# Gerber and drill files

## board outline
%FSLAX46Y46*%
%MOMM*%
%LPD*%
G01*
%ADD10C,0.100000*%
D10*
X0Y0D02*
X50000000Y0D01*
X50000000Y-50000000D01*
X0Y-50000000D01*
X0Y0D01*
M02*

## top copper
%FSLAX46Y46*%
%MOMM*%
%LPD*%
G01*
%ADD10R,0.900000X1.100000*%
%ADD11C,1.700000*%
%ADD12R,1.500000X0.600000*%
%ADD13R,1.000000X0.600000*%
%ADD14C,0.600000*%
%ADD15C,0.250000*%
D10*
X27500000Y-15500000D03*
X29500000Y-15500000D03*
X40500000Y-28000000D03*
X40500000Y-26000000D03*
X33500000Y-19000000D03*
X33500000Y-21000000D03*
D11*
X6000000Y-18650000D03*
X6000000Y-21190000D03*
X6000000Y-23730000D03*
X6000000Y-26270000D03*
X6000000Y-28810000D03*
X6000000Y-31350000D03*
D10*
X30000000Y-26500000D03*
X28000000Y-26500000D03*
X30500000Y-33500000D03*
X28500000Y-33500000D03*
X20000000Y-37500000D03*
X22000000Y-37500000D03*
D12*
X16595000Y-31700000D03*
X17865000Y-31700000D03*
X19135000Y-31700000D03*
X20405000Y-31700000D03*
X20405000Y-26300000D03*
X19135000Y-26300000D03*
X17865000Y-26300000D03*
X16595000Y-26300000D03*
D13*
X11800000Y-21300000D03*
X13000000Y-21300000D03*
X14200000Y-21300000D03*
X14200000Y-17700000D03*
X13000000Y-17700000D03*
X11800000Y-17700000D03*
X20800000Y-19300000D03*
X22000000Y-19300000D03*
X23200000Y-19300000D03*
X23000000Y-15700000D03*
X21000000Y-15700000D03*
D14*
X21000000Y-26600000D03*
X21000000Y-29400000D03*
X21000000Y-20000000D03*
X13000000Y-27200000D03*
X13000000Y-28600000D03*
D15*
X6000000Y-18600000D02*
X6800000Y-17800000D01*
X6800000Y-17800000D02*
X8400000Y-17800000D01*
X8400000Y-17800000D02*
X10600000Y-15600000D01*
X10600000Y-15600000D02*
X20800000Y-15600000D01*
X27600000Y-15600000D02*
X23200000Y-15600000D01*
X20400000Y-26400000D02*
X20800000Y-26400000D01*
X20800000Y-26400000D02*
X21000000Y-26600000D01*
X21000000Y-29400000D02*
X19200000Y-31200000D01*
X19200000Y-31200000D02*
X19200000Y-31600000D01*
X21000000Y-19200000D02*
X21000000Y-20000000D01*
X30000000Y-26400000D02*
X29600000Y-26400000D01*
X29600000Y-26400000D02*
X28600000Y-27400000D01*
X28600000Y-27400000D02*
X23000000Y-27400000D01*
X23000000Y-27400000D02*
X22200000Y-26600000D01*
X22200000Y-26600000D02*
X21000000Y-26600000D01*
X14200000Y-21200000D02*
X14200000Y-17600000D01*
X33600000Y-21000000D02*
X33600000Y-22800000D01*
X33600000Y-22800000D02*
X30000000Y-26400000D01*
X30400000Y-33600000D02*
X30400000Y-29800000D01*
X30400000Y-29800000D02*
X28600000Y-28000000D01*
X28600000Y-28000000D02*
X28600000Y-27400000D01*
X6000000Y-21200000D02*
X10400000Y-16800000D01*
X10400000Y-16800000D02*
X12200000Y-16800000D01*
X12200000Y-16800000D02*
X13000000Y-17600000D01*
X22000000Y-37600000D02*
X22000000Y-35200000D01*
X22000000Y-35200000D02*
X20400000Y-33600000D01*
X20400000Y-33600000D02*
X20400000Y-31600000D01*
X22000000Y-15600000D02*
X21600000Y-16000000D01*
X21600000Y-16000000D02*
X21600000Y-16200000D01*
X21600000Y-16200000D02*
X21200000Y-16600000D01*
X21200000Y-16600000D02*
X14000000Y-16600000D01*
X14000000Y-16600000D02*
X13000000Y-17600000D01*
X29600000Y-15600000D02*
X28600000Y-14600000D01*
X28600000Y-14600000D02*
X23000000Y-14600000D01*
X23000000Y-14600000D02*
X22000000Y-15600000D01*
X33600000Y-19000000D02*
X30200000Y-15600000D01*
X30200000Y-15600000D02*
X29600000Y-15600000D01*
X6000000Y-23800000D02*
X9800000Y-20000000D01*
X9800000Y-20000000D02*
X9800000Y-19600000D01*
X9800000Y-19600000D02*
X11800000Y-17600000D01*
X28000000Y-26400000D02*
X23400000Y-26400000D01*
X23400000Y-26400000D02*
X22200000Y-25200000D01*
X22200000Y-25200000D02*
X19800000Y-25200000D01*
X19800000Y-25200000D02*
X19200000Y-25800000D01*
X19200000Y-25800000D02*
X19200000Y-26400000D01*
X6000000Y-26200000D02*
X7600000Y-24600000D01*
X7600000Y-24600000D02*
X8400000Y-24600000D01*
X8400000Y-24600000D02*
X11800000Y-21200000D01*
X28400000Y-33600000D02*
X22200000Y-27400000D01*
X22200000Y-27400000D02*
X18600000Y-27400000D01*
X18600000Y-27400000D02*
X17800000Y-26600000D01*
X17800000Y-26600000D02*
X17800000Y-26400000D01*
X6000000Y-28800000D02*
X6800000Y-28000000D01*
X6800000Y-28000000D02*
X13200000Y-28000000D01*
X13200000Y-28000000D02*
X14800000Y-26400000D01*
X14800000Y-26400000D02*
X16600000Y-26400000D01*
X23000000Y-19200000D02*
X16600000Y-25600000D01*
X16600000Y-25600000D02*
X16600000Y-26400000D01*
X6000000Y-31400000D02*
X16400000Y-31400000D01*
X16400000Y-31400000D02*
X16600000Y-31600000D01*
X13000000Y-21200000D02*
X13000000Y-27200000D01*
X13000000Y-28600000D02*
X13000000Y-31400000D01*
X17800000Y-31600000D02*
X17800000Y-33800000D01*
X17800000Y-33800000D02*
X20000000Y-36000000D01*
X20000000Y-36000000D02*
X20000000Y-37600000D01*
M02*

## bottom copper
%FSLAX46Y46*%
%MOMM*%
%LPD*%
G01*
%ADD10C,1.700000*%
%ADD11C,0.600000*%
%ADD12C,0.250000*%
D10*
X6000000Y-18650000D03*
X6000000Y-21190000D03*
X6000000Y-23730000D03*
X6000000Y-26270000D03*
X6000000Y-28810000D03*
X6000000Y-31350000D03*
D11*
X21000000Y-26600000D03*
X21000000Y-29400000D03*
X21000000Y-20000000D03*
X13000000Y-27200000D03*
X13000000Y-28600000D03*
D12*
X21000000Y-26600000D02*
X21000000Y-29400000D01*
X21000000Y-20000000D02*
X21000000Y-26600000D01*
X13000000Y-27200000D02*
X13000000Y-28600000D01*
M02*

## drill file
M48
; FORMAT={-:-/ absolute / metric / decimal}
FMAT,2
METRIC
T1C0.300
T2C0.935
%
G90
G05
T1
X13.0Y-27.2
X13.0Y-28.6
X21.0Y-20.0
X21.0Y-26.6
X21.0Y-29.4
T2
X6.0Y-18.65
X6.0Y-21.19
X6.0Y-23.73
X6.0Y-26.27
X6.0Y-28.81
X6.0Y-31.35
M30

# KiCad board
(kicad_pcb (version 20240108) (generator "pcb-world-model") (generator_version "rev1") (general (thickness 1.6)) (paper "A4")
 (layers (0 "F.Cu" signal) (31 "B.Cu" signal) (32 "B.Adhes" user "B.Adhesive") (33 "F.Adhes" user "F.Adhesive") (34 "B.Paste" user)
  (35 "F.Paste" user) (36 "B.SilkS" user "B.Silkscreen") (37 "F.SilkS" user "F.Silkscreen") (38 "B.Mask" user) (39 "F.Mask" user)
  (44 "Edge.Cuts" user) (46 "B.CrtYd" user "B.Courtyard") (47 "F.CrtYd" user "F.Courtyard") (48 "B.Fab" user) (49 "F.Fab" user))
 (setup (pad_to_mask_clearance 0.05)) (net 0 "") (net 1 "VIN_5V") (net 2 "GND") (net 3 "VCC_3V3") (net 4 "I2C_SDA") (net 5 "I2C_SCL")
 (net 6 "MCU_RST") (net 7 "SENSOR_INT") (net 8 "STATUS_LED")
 (gr_rect (start 0.0 0.0) (end 50.0000 50.0000) (stroke (width 0.1) (type default)) (fill none) (layer "Edge.Cuts"))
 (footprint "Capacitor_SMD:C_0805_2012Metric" (layer "F.Cu") (at 28.5000 15.5000 0)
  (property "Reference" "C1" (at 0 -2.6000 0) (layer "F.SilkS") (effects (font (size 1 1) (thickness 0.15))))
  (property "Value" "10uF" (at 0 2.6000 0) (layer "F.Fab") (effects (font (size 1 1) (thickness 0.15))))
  (pad "1" smd rect (at -1.0000 0.0000) (size 0.9000 1.1000) (layers "F.Cu" "F.Paste" "F.Mask") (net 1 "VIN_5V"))
  (pad "2" smd rect (at 1.0000 0.0000) (size 0.9000 1.1000) (layers "F.Cu" "F.Paste" "F.Mask") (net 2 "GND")))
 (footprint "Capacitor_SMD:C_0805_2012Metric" (layer "F.Cu") (at 40.5000 27.0000 90)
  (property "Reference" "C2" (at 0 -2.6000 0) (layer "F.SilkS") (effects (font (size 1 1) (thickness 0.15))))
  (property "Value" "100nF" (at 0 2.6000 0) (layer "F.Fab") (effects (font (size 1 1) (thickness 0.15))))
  (pad "1" smd rect (at -1.0000 0.0000) (size 0.9000 1.1000) (layers "F.Cu" "F.Paste" "F.Mask") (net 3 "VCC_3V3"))
  (pad "2" smd rect (at 1.0000 0.0000) (size 0.9000 1.1000) (layers "F.Cu" "F.Paste" "F.Mask") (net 2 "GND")))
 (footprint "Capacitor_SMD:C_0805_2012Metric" (layer "F.Cu") (at 33.5000 20.0000 270)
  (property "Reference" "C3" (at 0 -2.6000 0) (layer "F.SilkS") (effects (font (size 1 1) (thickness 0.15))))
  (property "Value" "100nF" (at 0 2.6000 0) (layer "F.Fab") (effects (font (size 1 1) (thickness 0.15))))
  (pad "1" smd rect (at -1.0000 0.0000) (size 0.9000 1.1000) (layers "F.Cu" "F.Paste" "F.Mask") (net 3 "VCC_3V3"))
  (pad "2" smd rect (at 1.0000 0.0000) (size 0.9000 1.1000) (layers "F.Cu" "F.Paste" "F.Mask") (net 2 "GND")))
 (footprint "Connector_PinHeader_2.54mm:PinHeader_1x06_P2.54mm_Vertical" (layer "F.Cu") (at 6.0000 25.0000 0) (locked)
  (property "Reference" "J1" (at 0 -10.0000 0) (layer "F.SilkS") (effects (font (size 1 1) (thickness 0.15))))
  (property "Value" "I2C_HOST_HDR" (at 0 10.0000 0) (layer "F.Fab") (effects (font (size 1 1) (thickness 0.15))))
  (pad "1" thru_hole circle (at 0.0000 -6.3500) (size 1.7000 1.7000) (drill 0.9350) (layers "*.Cu" "*.Mask") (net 1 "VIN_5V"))
  (pad "2" thru_hole circle (at 0.0000 -3.8100) (size 1.7000 1.7000) (drill 0.9350) (layers "*.Cu" "*.Mask") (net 2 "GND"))
  (pad "3" thru_hole circle (at 0.0000 -1.2700) (size 1.7000 1.7000) (drill 0.9350) (layers "*.Cu" "*.Mask") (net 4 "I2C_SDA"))
  (pad "4" thru_hole circle (at 0.0000 1.2700) (size 1.7000 1.7000) (drill 0.9350) (layers "*.Cu" "*.Mask") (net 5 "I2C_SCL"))
  (pad "5" thru_hole circle (at 0.0000 3.8100) (size 1.7000 1.7000) (drill 0.9350) (layers "*.Cu" "*.Mask") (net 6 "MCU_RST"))
  (pad "6" thru_hole circle (at 0.0000 6.3500) (size 1.7000 1.7000) (drill 0.9350) (layers "*.Cu" "*.Mask") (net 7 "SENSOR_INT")))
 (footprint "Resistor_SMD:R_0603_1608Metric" (layer "F.Cu") (at 29.0000 26.5000 180)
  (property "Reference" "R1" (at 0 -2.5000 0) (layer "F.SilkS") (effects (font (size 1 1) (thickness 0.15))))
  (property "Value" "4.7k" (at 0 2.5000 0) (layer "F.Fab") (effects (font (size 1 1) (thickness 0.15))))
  (pad "1" smd rect (at -1.0000 0.0000) (size 0.9000 1.1000) (layers "F.Cu" "F.Paste" "F.Mask") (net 3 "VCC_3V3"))
  (pad "2" smd rect (at 1.0000 0.0000) (size 0.9000 1.1000) (layers "F.Cu" "F.Paste" "F.Mask") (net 4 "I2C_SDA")))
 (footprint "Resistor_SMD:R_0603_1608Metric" (layer "F.Cu") (at 29.5000 33.5000 180)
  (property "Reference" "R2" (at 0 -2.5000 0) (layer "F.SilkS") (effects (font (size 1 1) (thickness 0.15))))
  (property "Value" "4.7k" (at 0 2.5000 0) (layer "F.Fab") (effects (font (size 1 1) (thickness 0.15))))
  (pad "1" smd rect (at -1.0000 0.0000) (size 0.9000 1.1000) (layers "F.Cu" "F.Paste" "F.Mask") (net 3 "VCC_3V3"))
  (pad "2" smd rect (at 1.0000 0.0000) (size 0.9000 1.1000) (layers "F.Cu" "F.Paste" "F.Mask") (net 5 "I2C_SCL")))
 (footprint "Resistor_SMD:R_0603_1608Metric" (layer "F.Cu") (at 21.0000 37.5000 0)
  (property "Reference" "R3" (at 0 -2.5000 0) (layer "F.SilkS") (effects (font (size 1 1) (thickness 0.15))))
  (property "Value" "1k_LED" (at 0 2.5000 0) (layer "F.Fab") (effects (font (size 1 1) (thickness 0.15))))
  (pad "1" smd rect (at -1.0000 0.0000) (size 0.9000 1.1000) (layers "F.Cu" "F.Paste" "F.Mask") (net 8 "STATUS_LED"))
  (pad "2" smd rect (at 1.0000 0.0000) (size 0.9000 1.1000) (layers "F.Cu" "F.Paste" "F.Mask") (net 2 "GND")))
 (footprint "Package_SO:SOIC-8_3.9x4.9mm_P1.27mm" (layer "F.Cu") (at 18.5000 29.0000 90)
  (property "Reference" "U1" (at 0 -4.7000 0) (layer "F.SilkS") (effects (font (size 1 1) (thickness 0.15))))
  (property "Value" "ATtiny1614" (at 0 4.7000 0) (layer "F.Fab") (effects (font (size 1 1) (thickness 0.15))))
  (pad "1" smd rect (at -2.7000 -1.9050) (size 1.5000 0.6000) (layers "F.Cu" "F.Paste" "F.Mask") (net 3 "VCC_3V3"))
  (pad "2" smd rect (at -2.7000 -0.6350) (size 1.5000 0.6000) (layers "F.Cu" "F.Paste" "F.Mask") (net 4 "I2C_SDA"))
  (pad "3" smd rect (at -2.7000 0.6350) (size 1.5000 0.6000) (layers "F.Cu" "F.Paste" "F.Mask") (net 5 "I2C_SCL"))
  (pad "4" smd rect (at -2.7000 1.9050) (size 1.5000 0.6000) (layers "F.Cu" "F.Paste" "F.Mask") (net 6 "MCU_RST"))
  (pad "5" smd rect (at 2.7000 1.9050) (size 1.5000 0.6000) (layers "F.Cu" "F.Paste" "F.Mask") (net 7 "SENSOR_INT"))
  (pad "6" smd rect (at 2.7000 0.6350) (size 1.5000 0.6000) (layers "F.Cu" "F.Paste" "F.Mask") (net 8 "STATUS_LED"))
  (pad "7" smd rect (at 2.7000 -0.6350) (size 1.5000 0.6000) (layers "F.Cu" "F.Paste" "F.Mask") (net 3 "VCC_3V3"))
  (pad "8" smd rect (at 2.7000 -1.9050) (size 1.5000 0.6000) (layers "F.Cu" "F.Paste" "F.Mask") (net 2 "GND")))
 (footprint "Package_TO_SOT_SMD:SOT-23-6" (layer "F.Cu") (at 13.0000 19.5000 90)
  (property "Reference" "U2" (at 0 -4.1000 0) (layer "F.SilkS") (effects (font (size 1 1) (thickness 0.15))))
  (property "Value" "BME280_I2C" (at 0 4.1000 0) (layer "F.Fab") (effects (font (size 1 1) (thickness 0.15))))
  (pad "1" smd rect (at -1.8000 -1.2000) (size 1.0000 0.6000) (layers "F.Cu" "F.Paste" "F.Mask") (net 3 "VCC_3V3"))
  (pad "2" smd rect (at -1.8000 0.0000) (size 1.0000 0.6000) (layers "F.Cu" "F.Paste" "F.Mask") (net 2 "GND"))
  (pad "3" smd rect (at -1.8000 1.2000) (size 1.0000 0.6000) (layers "F.Cu" "F.Paste" "F.Mask") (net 4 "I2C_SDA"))
  (pad "4" smd rect (at 1.8000 1.2000) (size 1.0000 0.6000) (layers "F.Cu" "F.Paste" "F.Mask") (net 5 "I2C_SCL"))
  (pad "5" smd rect (at 1.8000 0.0000) (size 1.0000 0.6000) (layers "F.Cu" "F.Paste" "F.Mask") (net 7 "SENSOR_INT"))
  (pad "6" smd rect (at 1.8000 -1.2000) (size 1.0000 0.6000) (layers "F.Cu" "F.Paste" "F.Mask") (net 3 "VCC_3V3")))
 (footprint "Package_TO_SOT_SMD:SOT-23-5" (layer "F.Cu") (at 22.0000 17.5000 90)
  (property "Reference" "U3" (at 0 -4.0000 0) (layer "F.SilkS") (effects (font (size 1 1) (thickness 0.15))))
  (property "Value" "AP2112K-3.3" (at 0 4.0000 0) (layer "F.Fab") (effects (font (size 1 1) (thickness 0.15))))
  (pad "1" smd rect (at -1.8000 -1.2000) (size 1.0000 0.6000) (layers "F.Cu" "F.Paste" "F.Mask") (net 1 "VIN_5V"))
  (pad "2" smd rect (at -1.8000 0.0000) (size 1.0000 0.6000) (layers "F.Cu" "F.Paste" "F.Mask") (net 2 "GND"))
  (pad "3" smd rect (at -1.8000 1.2000) (size 1.0000 0.6000) (layers "F.Cu" "F.Paste" "F.Mask") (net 1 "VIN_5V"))
  (pad "4" smd rect (at 1.8000 1.0000) (size 1.0000 0.6000) (layers "F.Cu" "F.Paste" "F.Mask") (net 3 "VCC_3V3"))
  (pad "5" smd rect (at 1.8000 -1.0000) (size 1.0000 0.6000) (layers "F.Cu" "F.Paste" "F.Mask") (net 6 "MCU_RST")))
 (segment (start 6.0000 18.6000) (end 6.8000 17.8000) (width 0.2500) (layer "F.Cu") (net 1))
 (segment (start 6.8000 17.8000) (end 8.4000 17.8000) (width 0.2500) (layer "F.Cu") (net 1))
 (segment (start 8.4000 17.8000) (end 10.6000 15.6000) (width 0.2500) (layer "F.Cu") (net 1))
 (segment (start 10.6000 15.6000) (end 20.8000 15.6000) (width 0.2500) (layer "F.Cu") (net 1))
 (segment (start 27.6000 15.6000) (end 23.2000 15.6000) (width 0.2500) (layer "F.Cu") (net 1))
 (segment (start 20.4000 26.4000) (end 20.8000 26.4000) (width 0.2500) (layer "F.Cu") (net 3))
 (segment (start 20.8000 26.4000) (end 21.0000 26.6000) (width 0.2500) (layer "F.Cu") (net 3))
 (segment (start 21.0000 26.6000) (end 21.0000 29.4000) (width 0.2500) (layer "B.Cu") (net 3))
 (segment (start 21.0000 29.4000) (end 19.2000 31.2000) (width 0.2500) (layer "F.Cu") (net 3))
 (segment (start 19.2000 31.2000) (end 19.2000 31.6000) (width 0.2500) (layer "F.Cu") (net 3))
 (segment (start 21.0000 19.2000) (end 21.0000 20.0000) (width 0.2500) (layer "F.Cu") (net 3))
 (segment (start 21.0000 20.0000) (end 21.0000 26.6000) (width 0.2500) (layer "B.Cu") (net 3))
 (segment (start 30.0000 26.4000) (end 29.6000 26.4000) (width 0.2500) (layer "F.Cu") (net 3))
 (segment (start 29.6000 26.4000) (end 28.6000 27.4000) (width 0.2500) (layer "F.Cu") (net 3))
 (segment (start 28.6000 27.4000) (end 23.0000 27.4000) (width 0.2500) (layer "F.Cu") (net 3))
 (segment (start 23.0000 27.4000) (end 22.2000 26.6000) (width 0.2500) (layer "F.Cu") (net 3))
 (segment (start 22.2000 26.6000) (end 21.0000 26.6000) (width 0.2500) (layer "F.Cu") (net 3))
 (segment (start 14.2000 21.2000) (end 14.2000 17.6000) (width 0.2500) (layer "F.Cu") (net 3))
 (segment (start 33.6000 21.0000) (end 33.6000 22.8000) (width 0.2500) (layer "F.Cu") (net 3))
 (segment (start 33.6000 22.8000) (end 30.0000 26.4000) (width 0.2500) (layer "F.Cu") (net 3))
 (segment (start 30.4000 33.6000) (end 30.4000 29.8000) (width 0.2500) (layer "F.Cu") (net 3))
 (segment (start 30.4000 29.8000) (end 28.6000 28.0000) (width 0.2500) (layer "F.Cu") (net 3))
 (segment (start 28.6000 28.0000) (end 28.6000 27.4000) (width 0.2500) (layer "F.Cu") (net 3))
 (segment (start 6.0000 21.2000) (end 10.4000 16.8000) (width 0.2500) (layer "F.Cu") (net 2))
 (segment (start 10.4000 16.8000) (end 12.2000 16.8000) (width 0.2500) (layer "F.Cu") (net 2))
 (segment (start 12.2000 16.8000) (end 13.0000 17.6000) (width 0.2500) (layer "F.Cu") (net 2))
 (segment (start 22.0000 37.6000) (end 22.0000 35.2000) (width 0.2500) (layer "F.Cu") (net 2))
 (segment (start 22.0000 35.2000) (end 20.4000 33.6000) (width 0.2500) (layer "F.Cu") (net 2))
 (segment (start 20.4000 33.6000) (end 20.4000 31.6000) (width 0.2500) (layer "F.Cu") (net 2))
 (segment (start 22.0000 15.6000) (end 21.6000 16.0000) (width 0.2500) (layer "F.Cu") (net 2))
 (segment (start 21.6000 16.0000) (end 21.6000 16.2000) (width 0.2500) (layer "F.Cu") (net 2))
 (segment (start 21.6000 16.2000) (end 21.2000 16.6000) (width 0.2500) (layer "F.Cu") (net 2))
 (segment (start 21.2000 16.6000) (end 14.0000 16.6000) (width 0.2500) (layer "F.Cu") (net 2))
 (segment (start 14.0000 16.6000) (end 13.0000 17.6000) (width 0.2500) (layer "F.Cu") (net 2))
 (segment (start 29.6000 15.6000) (end 28.6000 14.6000) (width 0.2500) (layer "F.Cu") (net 2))
 (segment (start 28.6000 14.6000) (end 23.0000 14.6000) (width 0.2500) (layer "F.Cu") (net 2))
 (segment (start 23.0000 14.6000) (end 22.0000 15.6000) (width 0.2500) (layer "F.Cu") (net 2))
 (segment (start 33.6000 19.0000) (end 30.2000 15.6000) (width 0.2500) (layer "F.Cu") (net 2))
 (segment (start 30.2000 15.6000) (end 29.6000 15.6000) (width 0.2500) (layer "F.Cu") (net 2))
 (segment (start 6.0000 23.8000) (end 9.8000 20.0000) (width 0.2500) (layer "F.Cu") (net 4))
 (segment (start 9.8000 20.0000) (end 9.8000 19.6000) (width 0.2500) (layer "F.Cu") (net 4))
 (segment (start 9.8000 19.6000) (end 11.8000 17.6000) (width 0.2500) (layer "F.Cu") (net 4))
 (segment (start 28.0000 26.4000) (end 23.4000 26.4000) (width 0.2500) (layer "F.Cu") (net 4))
 (segment (start 23.4000 26.4000) (end 22.2000 25.2000) (width 0.2500) (layer "F.Cu") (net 4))
 (segment (start 22.2000 25.2000) (end 19.8000 25.2000) (width 0.2500) (layer "F.Cu") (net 4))
 (segment (start 19.8000 25.2000) (end 19.2000 25.8000) (width 0.2500) (layer "F.Cu") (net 4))
 (segment (start 19.2000 25.8000) (end 19.2000 26.4000) (width 0.2500) (layer "F.Cu") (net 4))
 (segment (start 6.0000 26.2000) (end 7.6000 24.6000) (width 0.2500) (layer "F.Cu") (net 5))
 (segment (start 7.6000 24.6000) (end 8.4000 24.6000) (width 0.2500) (layer "F.Cu") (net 5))
 (segment (start 8.4000 24.6000) (end 11.8000 21.2000) (width 0.2500) (layer "F.Cu") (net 5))
 (segment (start 28.4000 33.6000) (end 22.2000 27.4000) (width 0.2500) (layer "F.Cu") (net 5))
 (segment (start 22.2000 27.4000) (end 18.6000 27.4000) (width 0.2500) (layer "F.Cu") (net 5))
 (segment (start 18.6000 27.4000) (end 17.8000 26.6000) (width 0.2500) (layer "F.Cu") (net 5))
 (segment (start 17.8000 26.6000) (end 17.8000 26.4000) (width 0.2500) (layer "F.Cu") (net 5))
 (segment (start 6.0000 28.8000) (end 6.8000 28.0000) (width 0.2500) (layer "F.Cu") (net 6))
 (segment (start 6.8000 28.0000) (end 13.2000 28.0000) (width 0.2500) (layer "F.Cu") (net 6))
 (segment (start 13.2000 28.0000) (end 14.8000 26.4000) (width 0.2500) (layer "F.Cu") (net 6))
 (segment (start 14.8000 26.4000) (end 16.6000 26.4000) (width 0.2500) (layer "F.Cu") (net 6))
 (segment (start 23.0000 19.2000) (end 16.6000 25.6000) (width 0.2500) (layer "F.Cu") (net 6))
 (segment (start 16.6000 25.6000) (end 16.6000 26.4000) (width 0.2500) (layer "F.Cu") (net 6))
 (segment (start 6.0000 31.4000) (end 16.4000 31.4000) (width 0.2500) (layer "F.Cu") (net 7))
 (segment (start 16.4000 31.4000) (end 16.6000 31.6000) (width 0.2500) (layer "F.Cu") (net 7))
 (segment (start 13.0000 21.2000) (end 13.0000 27.2000) (width 0.2500) (layer "F.Cu") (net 7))
 (segment (start 13.0000 27.2000) (end 13.0000 28.6000) (width 0.2500) (layer "B.Cu") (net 7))
 (segment (start 13.0000 28.6000) (end 13.0000 31.4000) (width 0.2500) (layer "F.Cu") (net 7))
 (segment (start 17.8000 31.6000) (end 17.8000 33.8000) (width 0.2500) (layer "F.Cu") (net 8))
 (segment (start 17.8000 33.8000) (end 20.0000 36.0000) (width 0.2500) (layer "F.Cu") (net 8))
 (segment (start 20.0000 36.0000) (end 20.0000 37.6000) (width 0.2500) (layer "F.Cu") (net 8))
 (via (at 21.0000 26.6000) (size 0.6000) (drill 0.3000) (layers "F.Cu" "B.Cu") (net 3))
 (via (at 21.0000 29.4000) (size 0.6000) (drill 0.3000) (layers "F.Cu" "B.Cu") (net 3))
 (via (at 21.0000 20.0000) (size 0.6000) (drill 0.3000) (layers "F.Cu" "B.Cu") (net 3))
 (via (at 13.0000 27.2000) (size 0.6000) (drill 0.3000) (layers "F.Cu" "B.Cu") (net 7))
 (via (at 13.0000 28.6000) (size 0.6000) (drill 0.3000) (layers "F.Cu" "B.Cu") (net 7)))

